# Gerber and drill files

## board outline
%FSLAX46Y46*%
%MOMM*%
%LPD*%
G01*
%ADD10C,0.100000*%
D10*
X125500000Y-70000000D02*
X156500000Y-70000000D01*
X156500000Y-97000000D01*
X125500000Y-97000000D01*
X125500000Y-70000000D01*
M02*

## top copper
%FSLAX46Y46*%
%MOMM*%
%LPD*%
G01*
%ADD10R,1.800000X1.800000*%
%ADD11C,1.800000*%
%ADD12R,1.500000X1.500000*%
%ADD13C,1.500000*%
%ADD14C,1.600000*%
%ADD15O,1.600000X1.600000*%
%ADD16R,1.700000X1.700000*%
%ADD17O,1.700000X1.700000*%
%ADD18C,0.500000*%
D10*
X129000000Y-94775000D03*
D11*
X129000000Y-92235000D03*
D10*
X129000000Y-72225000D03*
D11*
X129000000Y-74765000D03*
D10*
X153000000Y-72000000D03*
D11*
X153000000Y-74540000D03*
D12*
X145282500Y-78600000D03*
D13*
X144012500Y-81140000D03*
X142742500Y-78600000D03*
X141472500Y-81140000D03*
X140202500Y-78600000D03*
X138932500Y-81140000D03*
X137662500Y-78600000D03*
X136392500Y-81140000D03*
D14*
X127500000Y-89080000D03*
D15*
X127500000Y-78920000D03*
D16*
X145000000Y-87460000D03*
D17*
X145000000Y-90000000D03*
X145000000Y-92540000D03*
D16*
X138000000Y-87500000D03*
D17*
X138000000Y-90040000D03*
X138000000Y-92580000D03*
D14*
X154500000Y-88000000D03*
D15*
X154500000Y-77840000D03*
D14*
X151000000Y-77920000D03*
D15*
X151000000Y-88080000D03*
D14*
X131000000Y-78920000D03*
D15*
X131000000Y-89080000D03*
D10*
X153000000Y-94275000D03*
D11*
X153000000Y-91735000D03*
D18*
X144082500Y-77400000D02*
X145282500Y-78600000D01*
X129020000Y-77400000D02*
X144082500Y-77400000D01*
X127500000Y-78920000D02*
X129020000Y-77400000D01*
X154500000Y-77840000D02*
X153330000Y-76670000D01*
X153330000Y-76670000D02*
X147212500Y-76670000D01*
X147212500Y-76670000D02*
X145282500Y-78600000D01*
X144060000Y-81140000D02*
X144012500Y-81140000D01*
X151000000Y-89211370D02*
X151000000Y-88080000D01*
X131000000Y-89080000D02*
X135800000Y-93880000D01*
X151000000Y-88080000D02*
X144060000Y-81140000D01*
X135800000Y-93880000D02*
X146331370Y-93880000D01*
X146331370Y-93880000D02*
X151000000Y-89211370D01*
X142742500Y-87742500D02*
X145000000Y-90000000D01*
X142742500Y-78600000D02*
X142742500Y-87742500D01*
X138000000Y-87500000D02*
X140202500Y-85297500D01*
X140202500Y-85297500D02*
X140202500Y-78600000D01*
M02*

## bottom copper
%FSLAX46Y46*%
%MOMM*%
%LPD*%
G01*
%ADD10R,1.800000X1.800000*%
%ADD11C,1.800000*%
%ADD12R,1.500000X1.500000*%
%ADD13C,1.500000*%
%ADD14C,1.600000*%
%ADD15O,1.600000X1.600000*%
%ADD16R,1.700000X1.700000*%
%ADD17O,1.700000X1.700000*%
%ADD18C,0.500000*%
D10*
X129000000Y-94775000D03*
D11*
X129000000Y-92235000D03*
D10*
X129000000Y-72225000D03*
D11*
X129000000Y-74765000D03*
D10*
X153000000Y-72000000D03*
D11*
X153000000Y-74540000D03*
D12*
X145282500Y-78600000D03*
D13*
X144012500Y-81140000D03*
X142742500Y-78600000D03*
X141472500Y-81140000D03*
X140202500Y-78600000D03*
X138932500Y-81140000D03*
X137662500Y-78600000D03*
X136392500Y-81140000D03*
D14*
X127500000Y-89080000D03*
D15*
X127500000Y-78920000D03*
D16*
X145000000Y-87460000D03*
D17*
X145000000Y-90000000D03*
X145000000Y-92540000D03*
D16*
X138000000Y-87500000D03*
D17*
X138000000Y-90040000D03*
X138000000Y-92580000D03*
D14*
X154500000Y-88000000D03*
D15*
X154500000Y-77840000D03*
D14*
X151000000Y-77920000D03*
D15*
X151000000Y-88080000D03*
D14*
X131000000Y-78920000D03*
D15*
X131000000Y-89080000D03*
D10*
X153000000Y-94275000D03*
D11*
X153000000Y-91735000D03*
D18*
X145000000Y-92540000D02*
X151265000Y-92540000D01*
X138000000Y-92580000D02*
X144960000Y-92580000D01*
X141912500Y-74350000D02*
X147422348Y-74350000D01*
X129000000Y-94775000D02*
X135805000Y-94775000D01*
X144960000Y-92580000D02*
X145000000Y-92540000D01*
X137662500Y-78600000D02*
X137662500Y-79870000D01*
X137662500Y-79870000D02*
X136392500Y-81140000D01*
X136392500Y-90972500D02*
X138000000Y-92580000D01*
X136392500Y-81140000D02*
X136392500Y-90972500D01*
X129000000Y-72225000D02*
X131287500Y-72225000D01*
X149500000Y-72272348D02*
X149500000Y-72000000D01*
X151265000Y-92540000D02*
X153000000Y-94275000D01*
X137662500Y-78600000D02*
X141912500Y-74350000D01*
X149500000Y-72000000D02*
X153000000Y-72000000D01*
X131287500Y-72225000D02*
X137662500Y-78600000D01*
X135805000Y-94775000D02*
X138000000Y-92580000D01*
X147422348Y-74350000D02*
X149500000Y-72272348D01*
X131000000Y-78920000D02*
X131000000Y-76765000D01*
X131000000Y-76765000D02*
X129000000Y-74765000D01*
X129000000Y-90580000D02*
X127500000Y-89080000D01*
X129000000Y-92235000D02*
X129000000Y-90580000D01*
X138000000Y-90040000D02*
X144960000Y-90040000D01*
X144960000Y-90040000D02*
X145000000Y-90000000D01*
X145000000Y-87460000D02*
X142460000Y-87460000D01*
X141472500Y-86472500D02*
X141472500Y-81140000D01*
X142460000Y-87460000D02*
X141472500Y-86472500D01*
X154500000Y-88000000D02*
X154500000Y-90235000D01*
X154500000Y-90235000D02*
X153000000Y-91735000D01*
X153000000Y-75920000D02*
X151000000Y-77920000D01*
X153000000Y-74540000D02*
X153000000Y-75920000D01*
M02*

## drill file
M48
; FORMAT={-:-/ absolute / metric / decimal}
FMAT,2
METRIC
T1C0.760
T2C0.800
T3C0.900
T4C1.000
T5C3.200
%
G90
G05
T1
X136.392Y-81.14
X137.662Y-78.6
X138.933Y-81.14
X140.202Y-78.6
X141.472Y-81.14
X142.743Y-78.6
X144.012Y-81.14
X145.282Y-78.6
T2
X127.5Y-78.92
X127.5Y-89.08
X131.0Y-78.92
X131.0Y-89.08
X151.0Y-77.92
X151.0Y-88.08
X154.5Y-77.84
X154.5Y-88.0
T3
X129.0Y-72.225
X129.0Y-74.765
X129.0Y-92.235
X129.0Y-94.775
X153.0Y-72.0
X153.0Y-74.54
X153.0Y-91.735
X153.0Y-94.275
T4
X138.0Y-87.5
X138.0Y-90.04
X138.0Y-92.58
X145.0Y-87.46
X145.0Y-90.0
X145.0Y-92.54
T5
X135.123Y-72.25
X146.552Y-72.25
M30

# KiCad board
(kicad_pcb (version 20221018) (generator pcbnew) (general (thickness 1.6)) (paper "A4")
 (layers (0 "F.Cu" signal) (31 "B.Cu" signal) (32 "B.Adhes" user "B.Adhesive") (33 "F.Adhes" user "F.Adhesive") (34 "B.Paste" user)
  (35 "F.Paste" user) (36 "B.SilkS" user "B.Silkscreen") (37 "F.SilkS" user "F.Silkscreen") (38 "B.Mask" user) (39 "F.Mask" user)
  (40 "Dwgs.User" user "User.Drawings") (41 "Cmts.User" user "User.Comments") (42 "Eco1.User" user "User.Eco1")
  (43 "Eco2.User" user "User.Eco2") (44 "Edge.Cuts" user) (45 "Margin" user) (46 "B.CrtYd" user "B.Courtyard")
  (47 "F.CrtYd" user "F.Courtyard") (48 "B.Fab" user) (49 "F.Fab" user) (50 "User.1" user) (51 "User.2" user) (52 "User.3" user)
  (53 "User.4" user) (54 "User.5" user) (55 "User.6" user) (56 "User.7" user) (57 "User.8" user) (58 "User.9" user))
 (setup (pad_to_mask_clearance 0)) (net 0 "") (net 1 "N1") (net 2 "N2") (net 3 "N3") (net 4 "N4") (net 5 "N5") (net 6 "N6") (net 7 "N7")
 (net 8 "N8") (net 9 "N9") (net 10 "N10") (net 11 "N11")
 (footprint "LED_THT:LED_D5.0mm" (layer "F.Cu") (at 129 94.775 90)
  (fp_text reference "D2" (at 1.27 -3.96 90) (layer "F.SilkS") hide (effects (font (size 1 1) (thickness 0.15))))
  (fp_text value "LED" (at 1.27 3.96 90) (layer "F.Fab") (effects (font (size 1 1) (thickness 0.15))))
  (pad "1" thru_hole rect (at 0 0 90) (size 1.8 1.8) (drill 0.9) (layers "*.Cu" "*.Mask") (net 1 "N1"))
  (pad "2" thru_hole circle (at 2.54 0 90) (size 1.8 1.8) (drill 0.9) (layers "*.Cu" "*.Mask") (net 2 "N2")))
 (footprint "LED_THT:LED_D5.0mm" (layer "F.Cu") (at 129 72.225 -90)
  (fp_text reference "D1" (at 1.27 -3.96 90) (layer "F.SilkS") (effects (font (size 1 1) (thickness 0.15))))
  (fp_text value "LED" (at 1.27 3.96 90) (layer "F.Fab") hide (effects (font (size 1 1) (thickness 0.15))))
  (pad "1" thru_hole rect (at 0 0 270) (size 1.8 1.8) (drill 0.9) (layers "*.Cu" "*.Mask") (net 1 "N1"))
  (pad "2" thru_hole circle (at 2.54 0 270) (size 1.8 1.8) (drill 0.9) (layers "*.Cu" "*.Mask") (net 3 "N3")))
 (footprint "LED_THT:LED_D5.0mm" (layer "F.Cu") (at 153 72 -90)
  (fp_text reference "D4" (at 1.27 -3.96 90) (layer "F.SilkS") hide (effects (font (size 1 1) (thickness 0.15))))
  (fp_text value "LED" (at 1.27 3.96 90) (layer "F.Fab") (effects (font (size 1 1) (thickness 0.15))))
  (pad "1" thru_hole rect (at 0 0 270) (size 1.8 1.8) (drill 0.9) (layers "*.Cu" "*.Mask") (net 1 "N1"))
  (pad "2" thru_hole circle (at 2.54 0 270) (size 1.8 1.8) (drill 0.9) (layers "*.Cu" "*.Mask") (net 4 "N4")))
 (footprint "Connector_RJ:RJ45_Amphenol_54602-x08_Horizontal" (layer "F.Cu") (at 145.2825 78.6 180)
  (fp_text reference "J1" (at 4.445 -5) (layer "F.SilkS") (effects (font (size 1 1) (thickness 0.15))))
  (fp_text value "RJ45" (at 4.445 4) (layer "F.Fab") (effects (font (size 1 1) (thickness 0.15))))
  (pad "" np_thru_hole circle (at -1.27 6.35 180) (size 3.2 3.2) (drill 3.2) (layers "*.Cu" "*.Mask"))
  (pad "" np_thru_hole circle (at 10.16 6.35 180) (size 3.2 3.2) (drill 3.2) (layers "*.Cu" "*.Mask"))
  (pad "1" thru_hole rect (at 0 0 180) (size 1.5 1.5) (drill 0.76) (layers "*.Cu" "*.Mask") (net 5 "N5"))
  (pad "2" thru_hole circle (at 1.27 -2.54 180) (size 1.5 1.5) (drill 0.76) (layers "*.Cu" "*.Mask") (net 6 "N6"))
  (pad "3" thru_hole circle (at 2.54 0 180) (size 1.5 1.5) (drill 0.76) (layers "*.Cu" "*.Mask") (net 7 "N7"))
  (pad "4" thru_hole circle (at 3.81 -2.54 180) (size 1.5 1.5) (drill 0.76) (layers "*.Cu" "*.Mask") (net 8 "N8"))
  (pad "5" thru_hole circle (at 5.08 0 180) (size 1.5 1.5) (drill 0.76) (layers "*.Cu" "*.Mask") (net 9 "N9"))
  (pad "6" thru_hole circle (at 6.35 -2.54 180) (size 1.5 1.5) (drill 0.76) (layers "*.Cu" "*.Mask") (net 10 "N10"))
  (pad "7" thru_hole circle (at 7.62 0 180) (size 1.5 1.5) (drill 0.76) (layers "*.Cu" "*.Mask") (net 1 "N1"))
  (pad "8" thru_hole circle (at 8.89 -2.54 180) (size 1.5 1.5) (drill 0.76) (layers "*.Cu" "*.Mask") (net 1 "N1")))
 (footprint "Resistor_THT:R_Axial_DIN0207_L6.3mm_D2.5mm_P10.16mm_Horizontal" (layer "F.Cu") (at 127.5 89.08 90)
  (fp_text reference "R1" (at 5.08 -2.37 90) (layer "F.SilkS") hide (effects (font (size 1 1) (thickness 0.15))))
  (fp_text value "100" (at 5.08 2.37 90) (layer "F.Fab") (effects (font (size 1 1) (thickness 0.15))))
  (pad "1" thru_hole circle (at 0 0 90) (size 1.6 1.6) (drill 0.8) (layers "*.Cu" "*.Mask") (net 2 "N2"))
  (pad "2" thru_hole oval (at 10.16 0 90) (size 1.6 1.6) (drill 0.8) (layers "*.Cu" "*.Mask") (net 5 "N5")))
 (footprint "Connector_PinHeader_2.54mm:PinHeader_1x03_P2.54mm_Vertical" (layer "F.Cu") (at 145 87.46)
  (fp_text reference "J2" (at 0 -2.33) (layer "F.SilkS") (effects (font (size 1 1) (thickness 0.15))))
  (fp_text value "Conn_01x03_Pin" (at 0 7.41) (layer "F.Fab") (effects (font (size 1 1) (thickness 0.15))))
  (pad "1" thru_hole rect (at 0 0) (size 1.7 1.7) (drill 1) (layers "*.Cu" "*.Mask") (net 8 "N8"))
  (pad "2" thru_hole oval (at 0 2.54) (size 1.7 1.7) (drill 1) (layers "*.Cu" "*.Mask") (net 7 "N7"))
  (pad "3" thru_hole oval (at 0 5.08) (size 1.7 1.7) (drill 1) (layers "*.Cu" "*.Mask") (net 1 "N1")))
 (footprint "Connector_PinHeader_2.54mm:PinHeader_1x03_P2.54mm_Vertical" (layer "F.Cu") (at 138 87.5)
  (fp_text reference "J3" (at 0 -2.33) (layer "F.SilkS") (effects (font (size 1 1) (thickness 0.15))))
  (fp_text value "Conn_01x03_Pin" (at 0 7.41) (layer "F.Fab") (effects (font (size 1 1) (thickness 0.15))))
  (pad "1" thru_hole rect (at 0 0) (size 1.7 1.7) (drill 1) (layers "*.Cu" "*.Mask") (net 9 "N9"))
  (pad "2" thru_hole oval (at 0 2.54) (size 1.7 1.7) (drill 1) (layers "*.Cu" "*.Mask") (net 7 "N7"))
  (pad "3" thru_hole oval (at 0 5.08) (size 1.7 1.7) (drill 1) (layers "*.Cu" "*.Mask") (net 1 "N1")))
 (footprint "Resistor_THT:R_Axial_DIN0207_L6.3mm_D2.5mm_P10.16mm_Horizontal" (layer "F.Cu") (at 154.5 88 90)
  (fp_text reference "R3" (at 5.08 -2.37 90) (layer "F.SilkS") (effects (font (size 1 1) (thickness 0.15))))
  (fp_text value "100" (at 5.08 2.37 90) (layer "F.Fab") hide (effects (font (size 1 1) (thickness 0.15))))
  (pad "1" thru_hole circle (at 0 0 90) (size 1.6 1.6) (drill 0.8) (layers "*.Cu" "*.Mask") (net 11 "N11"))
  (pad "2" thru_hole oval (at 10.16 0 90) (size 1.6 1.6) (drill 0.8) (layers "*.Cu" "*.Mask") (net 5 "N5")))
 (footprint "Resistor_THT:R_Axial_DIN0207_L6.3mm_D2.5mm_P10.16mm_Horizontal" (layer "F.Cu") (at 151 77.92 -90)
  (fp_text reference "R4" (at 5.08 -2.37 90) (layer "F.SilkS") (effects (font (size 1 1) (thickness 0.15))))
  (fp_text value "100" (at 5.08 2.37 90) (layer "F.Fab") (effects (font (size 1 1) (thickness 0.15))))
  (pad "1" thru_hole circle (at 0 0 270) (size 1.6 1.6) (drill 0.8) (layers "*.Cu" "*.Mask") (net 4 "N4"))
  (pad "2" thru_hole oval (at 10.16 0 270) (size 1.6 1.6) (drill 0.8) (layers "*.Cu" "*.Mask") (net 6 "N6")))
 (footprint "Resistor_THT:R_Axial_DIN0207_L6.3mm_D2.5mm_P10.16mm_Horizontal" (layer "F.Cu") (at 131 78.92 -90)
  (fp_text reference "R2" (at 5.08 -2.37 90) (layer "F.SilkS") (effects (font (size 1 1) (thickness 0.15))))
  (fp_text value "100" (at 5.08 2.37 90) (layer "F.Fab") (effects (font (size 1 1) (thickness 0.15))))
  (pad "1" thru_hole circle (at 0 0 270) (size 1.6 1.6) (drill 0.8) (layers "*.Cu" "*.Mask") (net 3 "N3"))
  (pad "2" thru_hole oval (at 10.16 0 270) (size 1.6 1.6) (drill 0.8) (layers "*.Cu" "*.Mask") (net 6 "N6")))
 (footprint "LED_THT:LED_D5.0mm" (layer "F.Cu") (at 153 94.275 90)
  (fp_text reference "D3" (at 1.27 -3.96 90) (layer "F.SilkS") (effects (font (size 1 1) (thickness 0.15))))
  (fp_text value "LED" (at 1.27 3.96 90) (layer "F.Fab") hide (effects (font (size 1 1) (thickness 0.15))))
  (pad "1" thru_hole rect (at 0 0 90) (size 1.8 1.8) (drill 0.9) (layers "*.Cu" "*.Mask") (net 1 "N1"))
  (pad "2" thru_hole circle (at 2.54 0 90) (size 1.8 1.8) (drill 0.9) (layers "*.Cu" "*.Mask") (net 11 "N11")))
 (gr_rect (start 125.5 70) (end 156.5 97) (stroke (width 0.1) (type default)) (fill none) (layer "Edge.Cuts"))
 (segment (start 145 92.54) (end 151.265 92.54) (width 0.5) (layer "B.Cu") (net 1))
 (segment (start 138 92.58) (end 144.96 92.58) (width 0.5) (layer "B.Cu") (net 1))
 (segment (start 141.9125 74.35) (end 147.422348 74.35) (width 0.5) (layer "B.Cu") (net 1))
 (segment (start 129 94.775) (end 135.805 94.775) (width 0.5) (layer "B.Cu") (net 1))
 (segment (start 144.96 92.58) (end 145 92.54) (width 0.5) (layer "B.Cu") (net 1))
 (segment (start 137.6625 78.6) (end 137.6625 79.87) (width 0.5) (layer "B.Cu") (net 1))
 (segment (start 137.6625 79.87) (end 136.3925 81.14) (width 0.5) (layer "B.Cu") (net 1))
 (segment (start 136.3925 90.9725) (end 138 92.58) (width 0.5) (layer "B.Cu") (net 1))
 (segment (start 136.3925 81.14) (end 136.3925 90.9725) (width 0.5) (layer "B.Cu") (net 1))
 (segment (start 129 72.225) (end 131.2875 72.225) (width 0.5) (layer "B.Cu") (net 1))
 (segment (start 149.5 72.272348) (end 149.5 72) (width 0.5) (layer "B.Cu") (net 1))
 (segment (start 151.265 92.54) (end 153 94.275) (width 0.5) (layer "B.Cu") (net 1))
 (segment (start 137.6625 78.6) (end 141.9125 74.35) (width 0.5) (layer "B.Cu") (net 1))
 (segment (start 149.5 72) (end 153 72) (width 0.5) (layer "B.Cu") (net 1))
 (segment (start 131.2875 72.225) (end 137.6625 78.6) (width 0.5) (layer "B.Cu") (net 1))
 (segment (start 135.805 94.775) (end 138 92.58) (width 0.5) (layer "B.Cu") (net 1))
 (segment (start 147.422348 74.35) (end 149.5 72.272348) (width 0.5) (layer "B.Cu") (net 1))
 (segment (start 131 78.92) (end 131 76.765) (width 0.5) (layer "B.Cu") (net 3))
 (segment (start 131 76.765) (end 129 74.765) (width 0.5) (layer "B.Cu") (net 3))
 (segment (start 129 90.58) (end 127.5 89.08) (width 0.5) (layer "B.Cu") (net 2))
 (segment (start 129 92.235) (end 129 90.58) (width 0.5) (layer "B.Cu") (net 2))
 (segment (start 144.0825 77.4) (end 145.2825 78.6) (width 0.5) (layer "F.Cu") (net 5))
 (segment (start 129.02 77.4) (end 144.0825 77.4) (width 0.5) (layer "F.Cu") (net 5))
 (segment (start 127.5 78.92) (end 129.02 77.4) (width 0.5) (layer "F.Cu") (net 5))
 (segment (start 154.5 77.84) (end 153.33 76.67) (width 0.5) (layer "F.Cu") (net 5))
 (segment (start 153.33 76.67) (end 147.2125 76.67) (width 0.5) (layer "F.Cu") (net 5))
 (segment (start 147.2125 76.67) (end 145.2825 78.6) (width 0.5) (layer "F.Cu") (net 5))
 (segment (start 144.06 81.14) (end 144.0125 81.14) (width 0.5) (layer "F.Cu") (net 6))
 (segment (start 151 89.21137) (end 151 88.08) (width 0.5) (layer "F.Cu") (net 6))
 (segment (start 131 89.08) (end 135.8 93.88) (width 0.5) (layer "F.Cu") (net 6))
 (segment (start 151 88.08) (end 144.06 81.14) (width 0.5) (layer "F.Cu") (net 6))
 (segment (start 135.8 93.88) (end 146.33137 93.88) (width 0.5) (layer "F.Cu") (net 6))
 (segment (start 146.33137 93.88) (end 151 89.21137) (width 0.5) (layer "F.Cu") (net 6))
 (segment (start 142.7425 87.7425) (end 145 90) (width 0.5) (layer "F.Cu") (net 7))
 (segment (start 142.7425 78.6) (end 142.7425 87.7425) (width 0.5) (layer "F.Cu") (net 7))
 (segment (start 138 90.04) (end 144.96 90.04) (width 0.5) (layer "B.Cu") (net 7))
 (segment (start 144.96 90.04) (end 145 90) (width 0.5) (layer "B.Cu") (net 7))
 (segment (start 145 87.46) (end 142.46 87.46) (width 0.5) (layer "B.Cu") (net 8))
 (segment (start 141.4725 86.4725) (end 141.4725 81.14) (width 0.5) (layer "B.Cu") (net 8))
 (segment (start 142.46 87.46) (end 141.4725 86.4725) (width 0.5) (layer "B.Cu") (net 8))
 (segment (start 138 87.5) (end 140.2025 85.2975) (width 0.5) (layer "F.Cu") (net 9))
 (segment (start 140.2025 85.2975) (end 140.2025 78.6) (width 0.5) (layer "F.Cu") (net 9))
 (segment (start 154.5 88) (end 154.5 90.235) (width 0.5) (layer "B.Cu") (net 11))
 (segment (start 154.5 90.235) (end 153 91.735) (width 0.5) (layer "B.Cu") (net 11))
 (segment (start 153 75.92) (end 151 77.92) (width 0.5) (layer "B.Cu") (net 4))
 (segment (start 153 74.54) (end 153 75.92) (width 0.5) (layer "B.Cu") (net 4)))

